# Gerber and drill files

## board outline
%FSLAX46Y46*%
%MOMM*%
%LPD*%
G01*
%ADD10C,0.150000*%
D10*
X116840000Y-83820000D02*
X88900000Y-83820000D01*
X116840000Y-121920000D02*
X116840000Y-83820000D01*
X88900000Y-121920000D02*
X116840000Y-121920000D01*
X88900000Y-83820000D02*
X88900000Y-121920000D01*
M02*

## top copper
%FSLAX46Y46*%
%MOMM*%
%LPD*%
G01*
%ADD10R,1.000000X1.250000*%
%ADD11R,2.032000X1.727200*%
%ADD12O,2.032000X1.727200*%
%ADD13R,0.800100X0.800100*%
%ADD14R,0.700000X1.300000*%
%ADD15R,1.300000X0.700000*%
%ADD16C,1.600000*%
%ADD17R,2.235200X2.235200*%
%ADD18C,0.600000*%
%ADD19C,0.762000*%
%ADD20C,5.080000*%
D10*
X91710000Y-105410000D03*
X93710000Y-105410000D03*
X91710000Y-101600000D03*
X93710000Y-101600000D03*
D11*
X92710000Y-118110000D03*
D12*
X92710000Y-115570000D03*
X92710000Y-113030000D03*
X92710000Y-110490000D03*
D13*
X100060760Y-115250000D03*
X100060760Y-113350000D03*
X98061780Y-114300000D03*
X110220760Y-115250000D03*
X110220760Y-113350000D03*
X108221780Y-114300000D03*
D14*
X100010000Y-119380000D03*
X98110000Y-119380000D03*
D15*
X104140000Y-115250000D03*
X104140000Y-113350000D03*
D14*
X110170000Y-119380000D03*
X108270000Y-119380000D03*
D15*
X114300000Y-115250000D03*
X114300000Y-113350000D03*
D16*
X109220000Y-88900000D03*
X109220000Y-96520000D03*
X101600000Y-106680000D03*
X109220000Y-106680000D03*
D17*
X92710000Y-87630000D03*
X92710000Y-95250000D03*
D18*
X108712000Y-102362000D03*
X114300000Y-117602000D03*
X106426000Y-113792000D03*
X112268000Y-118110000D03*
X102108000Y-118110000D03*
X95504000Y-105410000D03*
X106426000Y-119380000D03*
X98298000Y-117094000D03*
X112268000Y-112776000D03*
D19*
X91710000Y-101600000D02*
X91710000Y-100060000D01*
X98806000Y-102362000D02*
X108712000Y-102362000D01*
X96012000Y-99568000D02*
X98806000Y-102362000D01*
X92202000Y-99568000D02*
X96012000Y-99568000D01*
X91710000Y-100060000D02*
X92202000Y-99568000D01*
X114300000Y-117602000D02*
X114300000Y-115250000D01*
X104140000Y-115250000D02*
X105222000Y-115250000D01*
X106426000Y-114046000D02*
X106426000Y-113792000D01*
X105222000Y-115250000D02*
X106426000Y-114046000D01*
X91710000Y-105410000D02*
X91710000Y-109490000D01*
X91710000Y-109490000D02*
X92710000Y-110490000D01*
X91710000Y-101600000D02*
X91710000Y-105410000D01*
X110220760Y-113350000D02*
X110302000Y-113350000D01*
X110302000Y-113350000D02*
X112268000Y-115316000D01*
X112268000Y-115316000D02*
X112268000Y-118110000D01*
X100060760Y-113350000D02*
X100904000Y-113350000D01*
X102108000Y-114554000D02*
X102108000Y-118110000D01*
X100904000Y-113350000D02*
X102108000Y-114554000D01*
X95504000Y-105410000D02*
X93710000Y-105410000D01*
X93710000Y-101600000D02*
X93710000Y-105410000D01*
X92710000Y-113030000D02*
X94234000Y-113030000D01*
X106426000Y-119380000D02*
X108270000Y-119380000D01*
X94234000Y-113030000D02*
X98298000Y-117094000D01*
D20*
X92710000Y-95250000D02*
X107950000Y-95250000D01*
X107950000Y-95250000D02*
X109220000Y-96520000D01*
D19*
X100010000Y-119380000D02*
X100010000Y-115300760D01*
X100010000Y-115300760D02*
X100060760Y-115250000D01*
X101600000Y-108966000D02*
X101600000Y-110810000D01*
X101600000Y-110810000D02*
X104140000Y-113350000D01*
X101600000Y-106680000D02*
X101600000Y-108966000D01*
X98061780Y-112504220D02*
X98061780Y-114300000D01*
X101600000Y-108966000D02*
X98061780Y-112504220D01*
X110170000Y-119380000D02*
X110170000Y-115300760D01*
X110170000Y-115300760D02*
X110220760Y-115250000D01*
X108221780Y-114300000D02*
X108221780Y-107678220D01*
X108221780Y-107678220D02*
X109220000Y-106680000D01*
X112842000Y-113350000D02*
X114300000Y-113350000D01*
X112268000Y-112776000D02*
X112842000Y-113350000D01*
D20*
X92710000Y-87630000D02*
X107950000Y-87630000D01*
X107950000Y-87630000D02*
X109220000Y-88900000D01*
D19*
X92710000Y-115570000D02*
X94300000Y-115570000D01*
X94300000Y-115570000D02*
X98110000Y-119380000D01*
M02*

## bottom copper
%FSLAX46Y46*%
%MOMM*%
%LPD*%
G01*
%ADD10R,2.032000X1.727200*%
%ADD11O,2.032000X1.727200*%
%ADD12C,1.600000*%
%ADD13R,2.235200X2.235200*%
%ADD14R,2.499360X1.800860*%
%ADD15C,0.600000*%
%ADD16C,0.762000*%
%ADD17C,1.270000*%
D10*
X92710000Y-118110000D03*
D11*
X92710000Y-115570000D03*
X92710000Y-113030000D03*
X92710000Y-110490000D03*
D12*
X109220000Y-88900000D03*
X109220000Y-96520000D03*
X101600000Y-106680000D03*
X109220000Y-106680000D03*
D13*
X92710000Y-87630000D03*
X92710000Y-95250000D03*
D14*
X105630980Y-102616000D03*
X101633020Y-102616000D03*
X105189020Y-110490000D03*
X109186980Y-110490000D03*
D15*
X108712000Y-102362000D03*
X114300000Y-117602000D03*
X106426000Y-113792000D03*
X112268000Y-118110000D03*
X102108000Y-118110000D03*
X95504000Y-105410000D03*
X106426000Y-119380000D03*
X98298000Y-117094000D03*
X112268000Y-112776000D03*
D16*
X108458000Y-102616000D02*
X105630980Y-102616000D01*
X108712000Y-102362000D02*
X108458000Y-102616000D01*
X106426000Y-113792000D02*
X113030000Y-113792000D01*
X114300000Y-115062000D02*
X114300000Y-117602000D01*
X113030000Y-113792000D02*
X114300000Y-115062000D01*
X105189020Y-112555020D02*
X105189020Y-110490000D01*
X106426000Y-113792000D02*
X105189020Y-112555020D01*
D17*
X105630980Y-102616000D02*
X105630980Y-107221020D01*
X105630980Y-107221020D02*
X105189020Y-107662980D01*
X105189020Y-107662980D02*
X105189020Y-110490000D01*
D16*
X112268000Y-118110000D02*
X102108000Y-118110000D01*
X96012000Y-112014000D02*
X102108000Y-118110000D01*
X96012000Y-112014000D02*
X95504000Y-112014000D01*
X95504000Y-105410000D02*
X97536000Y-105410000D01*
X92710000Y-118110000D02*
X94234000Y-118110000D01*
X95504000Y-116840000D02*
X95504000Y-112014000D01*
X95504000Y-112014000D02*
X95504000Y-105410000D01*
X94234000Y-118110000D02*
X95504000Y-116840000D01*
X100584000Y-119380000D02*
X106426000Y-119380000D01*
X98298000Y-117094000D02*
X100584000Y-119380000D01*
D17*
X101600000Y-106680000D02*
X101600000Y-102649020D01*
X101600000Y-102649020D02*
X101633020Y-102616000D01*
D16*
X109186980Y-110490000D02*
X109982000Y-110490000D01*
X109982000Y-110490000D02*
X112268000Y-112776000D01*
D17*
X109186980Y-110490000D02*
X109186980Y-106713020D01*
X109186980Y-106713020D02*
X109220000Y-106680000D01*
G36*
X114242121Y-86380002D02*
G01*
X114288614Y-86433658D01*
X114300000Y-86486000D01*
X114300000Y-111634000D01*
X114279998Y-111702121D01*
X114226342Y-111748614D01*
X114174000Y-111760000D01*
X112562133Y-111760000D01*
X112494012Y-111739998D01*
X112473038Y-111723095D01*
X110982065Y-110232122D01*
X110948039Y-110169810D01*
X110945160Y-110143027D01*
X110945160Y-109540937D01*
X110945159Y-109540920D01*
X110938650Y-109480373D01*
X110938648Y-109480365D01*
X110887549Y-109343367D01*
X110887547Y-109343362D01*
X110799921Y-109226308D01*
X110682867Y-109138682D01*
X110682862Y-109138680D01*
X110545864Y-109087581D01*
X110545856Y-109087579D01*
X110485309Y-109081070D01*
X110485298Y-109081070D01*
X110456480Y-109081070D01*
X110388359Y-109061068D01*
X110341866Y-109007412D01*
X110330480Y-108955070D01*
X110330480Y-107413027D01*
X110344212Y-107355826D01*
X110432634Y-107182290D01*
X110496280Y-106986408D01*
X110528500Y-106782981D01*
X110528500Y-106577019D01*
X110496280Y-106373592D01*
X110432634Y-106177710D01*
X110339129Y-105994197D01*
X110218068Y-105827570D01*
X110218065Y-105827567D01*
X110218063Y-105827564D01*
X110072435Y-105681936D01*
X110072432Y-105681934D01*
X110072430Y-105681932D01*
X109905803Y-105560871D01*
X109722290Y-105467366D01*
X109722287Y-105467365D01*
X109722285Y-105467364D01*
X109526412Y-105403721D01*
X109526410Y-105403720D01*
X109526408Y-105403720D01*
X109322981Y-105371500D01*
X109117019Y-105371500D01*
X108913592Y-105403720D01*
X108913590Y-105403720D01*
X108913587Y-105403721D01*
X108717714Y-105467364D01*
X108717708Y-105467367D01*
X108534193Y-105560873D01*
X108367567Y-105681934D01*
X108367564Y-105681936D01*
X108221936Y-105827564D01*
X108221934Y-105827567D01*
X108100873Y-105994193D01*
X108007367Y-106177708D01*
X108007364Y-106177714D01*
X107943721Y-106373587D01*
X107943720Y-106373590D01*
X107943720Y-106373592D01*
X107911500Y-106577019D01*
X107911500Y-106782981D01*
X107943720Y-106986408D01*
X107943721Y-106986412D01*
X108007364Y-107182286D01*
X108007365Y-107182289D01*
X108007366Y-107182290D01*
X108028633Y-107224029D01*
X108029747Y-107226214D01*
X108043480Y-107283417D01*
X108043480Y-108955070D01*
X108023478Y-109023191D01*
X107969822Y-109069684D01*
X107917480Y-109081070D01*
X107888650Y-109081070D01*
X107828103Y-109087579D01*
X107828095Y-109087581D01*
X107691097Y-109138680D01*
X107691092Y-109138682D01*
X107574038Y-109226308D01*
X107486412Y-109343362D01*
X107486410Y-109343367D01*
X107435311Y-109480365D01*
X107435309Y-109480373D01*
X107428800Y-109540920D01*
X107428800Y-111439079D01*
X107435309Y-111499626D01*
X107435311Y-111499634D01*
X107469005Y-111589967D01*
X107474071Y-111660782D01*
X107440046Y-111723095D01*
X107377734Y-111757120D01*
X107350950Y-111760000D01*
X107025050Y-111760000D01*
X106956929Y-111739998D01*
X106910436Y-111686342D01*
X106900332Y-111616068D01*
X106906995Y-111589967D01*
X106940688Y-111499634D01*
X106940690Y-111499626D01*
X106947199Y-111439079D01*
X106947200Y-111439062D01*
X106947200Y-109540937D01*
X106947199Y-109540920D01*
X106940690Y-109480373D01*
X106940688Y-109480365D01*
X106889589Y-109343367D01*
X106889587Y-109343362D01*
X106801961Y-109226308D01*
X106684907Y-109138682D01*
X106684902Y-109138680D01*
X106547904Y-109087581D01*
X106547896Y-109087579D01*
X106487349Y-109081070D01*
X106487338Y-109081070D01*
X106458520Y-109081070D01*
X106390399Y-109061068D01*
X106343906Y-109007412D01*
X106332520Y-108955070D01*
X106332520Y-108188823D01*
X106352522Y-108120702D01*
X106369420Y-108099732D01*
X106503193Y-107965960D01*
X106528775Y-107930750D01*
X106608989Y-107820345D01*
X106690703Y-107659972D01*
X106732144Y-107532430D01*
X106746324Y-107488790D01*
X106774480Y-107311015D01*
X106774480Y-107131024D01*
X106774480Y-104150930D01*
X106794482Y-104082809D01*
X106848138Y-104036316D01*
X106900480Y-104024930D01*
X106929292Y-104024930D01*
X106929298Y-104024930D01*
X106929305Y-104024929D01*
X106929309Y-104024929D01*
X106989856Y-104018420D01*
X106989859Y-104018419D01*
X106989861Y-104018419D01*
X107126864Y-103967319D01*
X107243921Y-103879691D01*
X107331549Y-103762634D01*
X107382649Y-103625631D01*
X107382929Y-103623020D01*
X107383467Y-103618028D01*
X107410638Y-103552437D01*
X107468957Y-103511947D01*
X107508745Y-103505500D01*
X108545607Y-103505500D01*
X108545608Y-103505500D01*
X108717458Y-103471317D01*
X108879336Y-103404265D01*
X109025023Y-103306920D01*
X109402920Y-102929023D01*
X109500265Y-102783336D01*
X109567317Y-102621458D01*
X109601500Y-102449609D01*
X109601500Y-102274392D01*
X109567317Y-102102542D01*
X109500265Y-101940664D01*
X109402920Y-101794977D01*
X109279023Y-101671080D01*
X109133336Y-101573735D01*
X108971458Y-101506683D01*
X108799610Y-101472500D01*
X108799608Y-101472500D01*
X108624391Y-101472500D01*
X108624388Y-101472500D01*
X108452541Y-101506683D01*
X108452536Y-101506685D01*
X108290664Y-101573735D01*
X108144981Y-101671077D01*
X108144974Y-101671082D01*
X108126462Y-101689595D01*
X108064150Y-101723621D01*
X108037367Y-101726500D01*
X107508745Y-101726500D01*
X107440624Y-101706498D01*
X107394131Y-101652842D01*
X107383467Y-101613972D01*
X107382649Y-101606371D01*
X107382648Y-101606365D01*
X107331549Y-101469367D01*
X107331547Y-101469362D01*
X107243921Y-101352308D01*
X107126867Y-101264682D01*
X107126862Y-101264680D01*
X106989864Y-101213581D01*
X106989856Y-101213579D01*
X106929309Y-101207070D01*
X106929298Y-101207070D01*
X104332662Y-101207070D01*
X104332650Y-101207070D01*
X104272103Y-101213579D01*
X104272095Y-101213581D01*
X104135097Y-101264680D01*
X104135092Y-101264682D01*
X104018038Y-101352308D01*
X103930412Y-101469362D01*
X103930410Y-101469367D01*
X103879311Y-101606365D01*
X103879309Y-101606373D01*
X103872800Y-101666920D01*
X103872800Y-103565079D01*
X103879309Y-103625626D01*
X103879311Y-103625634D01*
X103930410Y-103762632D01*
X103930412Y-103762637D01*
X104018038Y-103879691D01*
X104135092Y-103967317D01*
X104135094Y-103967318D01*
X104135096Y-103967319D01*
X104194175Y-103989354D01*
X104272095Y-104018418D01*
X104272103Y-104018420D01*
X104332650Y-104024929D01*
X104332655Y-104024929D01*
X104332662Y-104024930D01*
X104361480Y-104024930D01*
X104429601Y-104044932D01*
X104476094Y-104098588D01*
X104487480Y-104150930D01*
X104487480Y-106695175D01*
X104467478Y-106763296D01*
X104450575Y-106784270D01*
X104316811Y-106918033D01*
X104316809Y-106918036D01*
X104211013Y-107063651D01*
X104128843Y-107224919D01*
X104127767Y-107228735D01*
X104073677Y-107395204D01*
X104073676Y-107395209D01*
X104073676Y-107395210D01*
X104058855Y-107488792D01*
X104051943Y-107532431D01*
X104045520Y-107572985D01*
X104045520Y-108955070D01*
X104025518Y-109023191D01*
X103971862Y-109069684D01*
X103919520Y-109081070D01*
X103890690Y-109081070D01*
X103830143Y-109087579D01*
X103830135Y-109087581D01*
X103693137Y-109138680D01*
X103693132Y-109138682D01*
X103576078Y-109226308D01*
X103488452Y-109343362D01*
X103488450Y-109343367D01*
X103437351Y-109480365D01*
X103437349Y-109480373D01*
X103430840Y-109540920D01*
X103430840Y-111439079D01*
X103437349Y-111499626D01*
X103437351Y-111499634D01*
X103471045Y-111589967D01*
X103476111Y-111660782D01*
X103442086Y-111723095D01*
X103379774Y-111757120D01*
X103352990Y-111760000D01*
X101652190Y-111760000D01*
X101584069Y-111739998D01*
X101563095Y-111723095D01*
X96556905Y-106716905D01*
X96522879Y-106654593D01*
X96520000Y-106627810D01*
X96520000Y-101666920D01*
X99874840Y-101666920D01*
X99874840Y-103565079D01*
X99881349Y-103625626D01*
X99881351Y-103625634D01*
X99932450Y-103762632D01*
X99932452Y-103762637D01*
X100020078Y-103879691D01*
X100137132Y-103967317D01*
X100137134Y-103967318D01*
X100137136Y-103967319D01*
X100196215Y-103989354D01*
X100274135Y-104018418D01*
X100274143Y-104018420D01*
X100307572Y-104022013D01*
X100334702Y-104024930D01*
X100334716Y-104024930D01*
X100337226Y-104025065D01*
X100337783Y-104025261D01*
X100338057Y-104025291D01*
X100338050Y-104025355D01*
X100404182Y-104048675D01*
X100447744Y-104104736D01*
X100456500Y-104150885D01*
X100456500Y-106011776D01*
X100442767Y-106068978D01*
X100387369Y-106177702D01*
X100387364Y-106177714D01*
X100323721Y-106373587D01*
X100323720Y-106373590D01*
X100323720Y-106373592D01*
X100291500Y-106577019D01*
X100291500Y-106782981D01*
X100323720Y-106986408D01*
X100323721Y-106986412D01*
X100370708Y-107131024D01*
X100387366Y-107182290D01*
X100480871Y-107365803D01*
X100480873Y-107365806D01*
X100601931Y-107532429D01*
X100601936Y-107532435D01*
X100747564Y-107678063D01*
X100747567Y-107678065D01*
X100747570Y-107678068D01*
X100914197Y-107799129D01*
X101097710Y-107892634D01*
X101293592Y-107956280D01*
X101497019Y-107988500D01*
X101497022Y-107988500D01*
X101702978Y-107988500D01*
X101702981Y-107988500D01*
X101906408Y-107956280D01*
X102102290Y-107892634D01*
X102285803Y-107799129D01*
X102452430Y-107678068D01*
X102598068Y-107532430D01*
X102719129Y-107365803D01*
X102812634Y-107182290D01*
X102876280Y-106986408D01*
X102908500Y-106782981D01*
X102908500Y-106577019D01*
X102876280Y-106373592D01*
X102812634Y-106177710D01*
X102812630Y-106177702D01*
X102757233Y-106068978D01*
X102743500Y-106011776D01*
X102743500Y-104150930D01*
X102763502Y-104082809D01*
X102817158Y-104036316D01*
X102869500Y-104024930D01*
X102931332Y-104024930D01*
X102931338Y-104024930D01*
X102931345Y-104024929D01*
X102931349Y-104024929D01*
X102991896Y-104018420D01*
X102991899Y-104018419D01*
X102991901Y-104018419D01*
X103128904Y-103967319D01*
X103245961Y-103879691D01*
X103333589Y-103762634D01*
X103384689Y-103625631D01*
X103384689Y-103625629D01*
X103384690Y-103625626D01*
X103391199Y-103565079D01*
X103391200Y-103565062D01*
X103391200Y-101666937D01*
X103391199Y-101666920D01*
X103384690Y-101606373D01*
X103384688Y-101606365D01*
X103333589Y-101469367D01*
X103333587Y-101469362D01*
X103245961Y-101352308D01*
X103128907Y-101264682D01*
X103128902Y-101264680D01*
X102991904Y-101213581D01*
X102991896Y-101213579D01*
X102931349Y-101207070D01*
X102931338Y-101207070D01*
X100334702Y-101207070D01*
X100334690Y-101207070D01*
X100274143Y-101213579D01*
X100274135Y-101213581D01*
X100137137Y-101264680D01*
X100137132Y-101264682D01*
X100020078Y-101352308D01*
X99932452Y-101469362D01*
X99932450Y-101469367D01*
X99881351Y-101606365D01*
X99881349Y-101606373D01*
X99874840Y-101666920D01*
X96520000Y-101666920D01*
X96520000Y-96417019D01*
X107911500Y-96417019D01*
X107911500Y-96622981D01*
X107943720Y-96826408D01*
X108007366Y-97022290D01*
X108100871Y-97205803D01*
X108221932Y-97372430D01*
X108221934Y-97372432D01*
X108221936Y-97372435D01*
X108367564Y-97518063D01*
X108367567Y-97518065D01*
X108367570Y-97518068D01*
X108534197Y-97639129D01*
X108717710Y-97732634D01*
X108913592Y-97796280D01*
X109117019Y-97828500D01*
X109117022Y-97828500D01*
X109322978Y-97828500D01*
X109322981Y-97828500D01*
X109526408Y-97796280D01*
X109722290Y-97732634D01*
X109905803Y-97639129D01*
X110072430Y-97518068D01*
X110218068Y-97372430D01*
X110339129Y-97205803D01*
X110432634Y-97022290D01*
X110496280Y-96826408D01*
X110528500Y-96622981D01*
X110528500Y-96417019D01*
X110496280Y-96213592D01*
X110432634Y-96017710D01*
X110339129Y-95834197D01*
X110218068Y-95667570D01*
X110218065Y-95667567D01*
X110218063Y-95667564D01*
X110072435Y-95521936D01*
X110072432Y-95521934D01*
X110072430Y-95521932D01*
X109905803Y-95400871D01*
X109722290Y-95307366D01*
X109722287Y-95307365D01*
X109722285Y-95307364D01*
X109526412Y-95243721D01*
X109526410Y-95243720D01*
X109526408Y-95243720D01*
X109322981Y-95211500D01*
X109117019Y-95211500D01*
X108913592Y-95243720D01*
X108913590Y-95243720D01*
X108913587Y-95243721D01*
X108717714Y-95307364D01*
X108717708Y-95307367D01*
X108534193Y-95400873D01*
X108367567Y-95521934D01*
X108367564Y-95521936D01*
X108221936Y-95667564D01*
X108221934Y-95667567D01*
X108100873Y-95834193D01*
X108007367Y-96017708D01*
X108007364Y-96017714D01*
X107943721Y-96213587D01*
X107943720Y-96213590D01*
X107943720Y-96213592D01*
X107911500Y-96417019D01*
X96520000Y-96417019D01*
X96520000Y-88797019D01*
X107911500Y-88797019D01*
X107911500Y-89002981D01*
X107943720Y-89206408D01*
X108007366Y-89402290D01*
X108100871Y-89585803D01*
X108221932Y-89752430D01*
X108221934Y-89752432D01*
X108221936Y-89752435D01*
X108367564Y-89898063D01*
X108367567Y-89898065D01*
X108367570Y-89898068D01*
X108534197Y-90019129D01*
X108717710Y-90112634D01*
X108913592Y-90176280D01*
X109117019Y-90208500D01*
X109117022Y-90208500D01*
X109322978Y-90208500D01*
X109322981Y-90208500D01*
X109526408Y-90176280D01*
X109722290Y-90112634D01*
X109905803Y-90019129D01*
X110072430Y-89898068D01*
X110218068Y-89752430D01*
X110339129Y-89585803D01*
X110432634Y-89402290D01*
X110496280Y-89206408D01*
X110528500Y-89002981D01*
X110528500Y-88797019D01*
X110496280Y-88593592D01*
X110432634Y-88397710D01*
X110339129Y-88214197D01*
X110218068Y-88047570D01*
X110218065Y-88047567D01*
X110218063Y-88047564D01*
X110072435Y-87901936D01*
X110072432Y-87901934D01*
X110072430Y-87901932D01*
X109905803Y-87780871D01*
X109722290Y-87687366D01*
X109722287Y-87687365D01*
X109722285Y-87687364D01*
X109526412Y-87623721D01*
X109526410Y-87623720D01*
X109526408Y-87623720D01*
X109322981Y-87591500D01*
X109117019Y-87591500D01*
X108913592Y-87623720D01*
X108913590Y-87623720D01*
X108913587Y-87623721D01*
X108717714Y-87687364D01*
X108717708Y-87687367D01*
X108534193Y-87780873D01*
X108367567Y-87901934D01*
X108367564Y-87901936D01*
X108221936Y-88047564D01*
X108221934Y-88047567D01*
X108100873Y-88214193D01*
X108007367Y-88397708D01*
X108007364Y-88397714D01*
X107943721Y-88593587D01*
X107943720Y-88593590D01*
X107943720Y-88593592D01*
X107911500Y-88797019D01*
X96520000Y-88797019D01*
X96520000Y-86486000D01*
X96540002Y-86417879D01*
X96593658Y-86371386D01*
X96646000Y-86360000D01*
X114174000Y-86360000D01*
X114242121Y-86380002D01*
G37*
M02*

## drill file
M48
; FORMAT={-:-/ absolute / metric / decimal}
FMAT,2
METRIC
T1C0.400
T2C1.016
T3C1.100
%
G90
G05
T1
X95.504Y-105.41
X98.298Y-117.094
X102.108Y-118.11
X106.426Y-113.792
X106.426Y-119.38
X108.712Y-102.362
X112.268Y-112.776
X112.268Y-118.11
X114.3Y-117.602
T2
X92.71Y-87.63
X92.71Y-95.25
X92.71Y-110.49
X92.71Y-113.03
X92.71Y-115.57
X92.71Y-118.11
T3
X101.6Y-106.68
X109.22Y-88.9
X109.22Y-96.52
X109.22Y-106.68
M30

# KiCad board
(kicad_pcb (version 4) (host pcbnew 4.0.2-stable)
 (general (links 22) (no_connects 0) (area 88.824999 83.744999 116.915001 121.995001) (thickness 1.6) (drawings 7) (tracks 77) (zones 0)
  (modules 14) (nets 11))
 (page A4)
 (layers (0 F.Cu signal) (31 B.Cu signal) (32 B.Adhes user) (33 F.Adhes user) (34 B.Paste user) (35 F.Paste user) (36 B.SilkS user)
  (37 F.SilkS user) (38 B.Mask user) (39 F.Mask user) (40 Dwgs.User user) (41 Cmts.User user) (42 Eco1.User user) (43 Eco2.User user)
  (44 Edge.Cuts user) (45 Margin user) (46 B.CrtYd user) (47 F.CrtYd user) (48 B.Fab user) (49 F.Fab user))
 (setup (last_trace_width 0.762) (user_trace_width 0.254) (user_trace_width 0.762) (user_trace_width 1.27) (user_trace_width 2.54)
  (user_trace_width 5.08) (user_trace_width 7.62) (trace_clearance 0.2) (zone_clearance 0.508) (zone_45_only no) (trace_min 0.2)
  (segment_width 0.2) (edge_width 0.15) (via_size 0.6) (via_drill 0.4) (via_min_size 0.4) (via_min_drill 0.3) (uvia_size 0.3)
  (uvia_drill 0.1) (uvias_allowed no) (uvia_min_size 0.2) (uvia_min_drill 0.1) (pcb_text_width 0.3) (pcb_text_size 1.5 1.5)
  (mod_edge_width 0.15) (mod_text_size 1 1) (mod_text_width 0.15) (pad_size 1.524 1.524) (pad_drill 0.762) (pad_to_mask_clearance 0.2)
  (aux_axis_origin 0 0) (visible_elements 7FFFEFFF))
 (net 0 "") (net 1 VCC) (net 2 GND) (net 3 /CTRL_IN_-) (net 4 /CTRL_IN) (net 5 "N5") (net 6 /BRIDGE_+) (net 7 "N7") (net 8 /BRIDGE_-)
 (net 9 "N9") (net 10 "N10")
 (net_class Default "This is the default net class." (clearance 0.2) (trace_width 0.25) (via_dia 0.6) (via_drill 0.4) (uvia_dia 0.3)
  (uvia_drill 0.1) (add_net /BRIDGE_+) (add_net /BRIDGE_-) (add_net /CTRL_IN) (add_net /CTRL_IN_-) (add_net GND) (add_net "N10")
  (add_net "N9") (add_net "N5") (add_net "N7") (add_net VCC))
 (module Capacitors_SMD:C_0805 (layer F.Cu) (at 92.71 105.41)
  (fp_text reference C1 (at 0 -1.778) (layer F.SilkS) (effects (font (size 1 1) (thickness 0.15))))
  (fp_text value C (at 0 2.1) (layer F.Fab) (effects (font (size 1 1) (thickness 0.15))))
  (pad 1 smd rect (at -1 0) (size 1 1.25) (layers F.Cu F.Paste F.Mask) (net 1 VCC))
  (pad 2 smd rect (at 1 0) (size 1 1.25) (layers F.Cu F.Paste F.Mask) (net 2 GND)))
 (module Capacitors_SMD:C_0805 (layer F.Cu) (at 92.71 101.6)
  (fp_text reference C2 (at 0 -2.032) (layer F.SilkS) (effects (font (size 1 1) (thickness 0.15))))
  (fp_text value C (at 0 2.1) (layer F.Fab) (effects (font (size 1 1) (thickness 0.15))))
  (pad 1 smd rect (at -1 0) (size 1 1.25) (layers F.Cu F.Paste F.Mask) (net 1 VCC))
  (pad 2 smd rect (at 1 0) (size 1 1.25) (layers F.Cu F.Paste F.Mask) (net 2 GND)))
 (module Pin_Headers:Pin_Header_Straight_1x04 (layer F.Cu) (at 92.71 118.11 180)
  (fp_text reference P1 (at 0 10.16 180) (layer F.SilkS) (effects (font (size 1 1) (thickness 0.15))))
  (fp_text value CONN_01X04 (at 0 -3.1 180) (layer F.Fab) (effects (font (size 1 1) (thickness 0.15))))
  (pad 1 thru_hole rect (at 0 0 180) (size 2.032 1.7272) (drill 1.016) (layers *.Cu *.Mask F.SilkS) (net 2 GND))
  (pad 2 thru_hole oval (at 0 2.54 180) (size 2.032 1.7272) (drill 1.016) (layers *.Cu *.Mask F.SilkS) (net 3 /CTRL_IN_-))
  (pad 3 thru_hole oval (at 0 5.08 180) (size 2.032 1.7272) (drill 1.016) (layers *.Cu *.Mask F.SilkS) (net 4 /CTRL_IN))
  (pad 4 thru_hole oval (at 0 7.62 180) (size 2.032 1.7272) (drill 1.016) (layers *.Cu *.Mask F.SilkS) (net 1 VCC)))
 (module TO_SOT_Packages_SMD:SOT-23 (layer F.Cu) (at 99.06 114.3 90)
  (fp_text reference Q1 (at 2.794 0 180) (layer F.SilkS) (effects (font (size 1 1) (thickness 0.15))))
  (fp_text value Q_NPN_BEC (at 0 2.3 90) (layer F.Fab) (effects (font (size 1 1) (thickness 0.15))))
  (pad 1 smd rect (at -0.95 1.00076 90) (size 0.8001 0.8001) (layers F.Cu F.Paste F.Mask) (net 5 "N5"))
  (pad 2 smd rect (at 0.95 1.00076 90) (size 0.8001 0.8001) (layers F.Cu F.Paste F.Mask) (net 2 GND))
  (pad 3 smd rect (at 0 -0.99822 90) (size 0.8001 0.8001) (layers F.Cu F.Paste F.Mask) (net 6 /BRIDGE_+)))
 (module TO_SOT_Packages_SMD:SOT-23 (layer F.Cu) (at 109.22 114.3 90)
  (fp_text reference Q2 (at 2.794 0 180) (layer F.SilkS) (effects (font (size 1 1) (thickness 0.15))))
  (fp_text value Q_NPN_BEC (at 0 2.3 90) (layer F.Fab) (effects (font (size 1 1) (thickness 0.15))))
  (pad 1 smd rect (at -0.95 1.00076 90) (size 0.8001 0.8001) (layers F.Cu F.Paste F.Mask) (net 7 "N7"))
  (pad 2 smd rect (at 0.95 1.00076 90) (size 0.8001 0.8001) (layers F.Cu F.Paste F.Mask) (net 2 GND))
  (pad 3 smd rect (at 0 -0.99822 90) (size 0.8001 0.8001) (layers F.Cu F.Paste F.Mask) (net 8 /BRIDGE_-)))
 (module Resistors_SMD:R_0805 (layer F.Cu) (at 99.06 119.38 180)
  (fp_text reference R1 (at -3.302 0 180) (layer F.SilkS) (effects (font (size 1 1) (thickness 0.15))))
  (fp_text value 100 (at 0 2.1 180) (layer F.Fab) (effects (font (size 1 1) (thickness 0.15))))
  (pad 1 smd rect (at -0.95 0 180) (size 0.7 1.3) (layers F.Cu F.Paste F.Mask) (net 5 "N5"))
  (pad 2 smd rect (at 0.95 0 180) (size 0.7 1.3) (layers F.Cu F.Paste F.Mask) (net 3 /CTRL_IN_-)))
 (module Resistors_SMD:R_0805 (layer F.Cu) (at 104.14 114.3 90)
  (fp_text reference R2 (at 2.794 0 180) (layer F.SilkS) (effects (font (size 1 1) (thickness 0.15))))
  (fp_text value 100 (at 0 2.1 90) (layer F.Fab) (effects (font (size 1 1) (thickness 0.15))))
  (pad 1 smd rect (at -0.95 0 90) (size 0.7 1.3) (layers F.Cu F.Paste F.Mask) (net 1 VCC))
  (pad 2 smd rect (at 0.95 0 90) (size 0.7 1.3) (layers F.Cu F.Paste F.Mask) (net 6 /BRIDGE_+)))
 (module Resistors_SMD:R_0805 (layer F.Cu) (at 109.22 119.38 180)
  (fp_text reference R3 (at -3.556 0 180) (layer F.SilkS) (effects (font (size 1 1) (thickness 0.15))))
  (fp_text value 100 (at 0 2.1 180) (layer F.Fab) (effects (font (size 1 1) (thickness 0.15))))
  (pad 1 smd rect (at -0.95 0 180) (size 0.7 1.3) (layers F.Cu F.Paste F.Mask) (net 7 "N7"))
  (pad 2 smd rect (at 0.95 0 180) (size 0.7 1.3) (layers F.Cu F.Paste F.Mask) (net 4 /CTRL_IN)))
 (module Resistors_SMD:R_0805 (layer F.Cu) (at 114.3 114.3 90)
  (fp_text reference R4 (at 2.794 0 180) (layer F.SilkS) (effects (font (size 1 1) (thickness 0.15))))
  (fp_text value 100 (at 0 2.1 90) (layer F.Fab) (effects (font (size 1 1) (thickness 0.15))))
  (pad 1 smd rect (at -0.95 0 90) (size 0.7 1.3) (layers F.Cu F.Paste F.Mask) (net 1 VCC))
  (pad 2 smd rect (at 0.95 0 90) (size 0.7 1.3) (layers F.Cu F.Paste F.Mask) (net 8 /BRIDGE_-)))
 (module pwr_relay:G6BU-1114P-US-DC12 (layer F.Cu) (at 109.22 106.68 90)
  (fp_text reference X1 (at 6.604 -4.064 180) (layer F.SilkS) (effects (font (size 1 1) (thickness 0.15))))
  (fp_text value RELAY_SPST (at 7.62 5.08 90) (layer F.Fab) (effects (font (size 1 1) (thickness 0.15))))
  (pad 4 thru_hole circle (at 17.78 0 90) (size 1.6 1.6) (drill 1.1) (layers *.Cu *.Mask F.SilkS) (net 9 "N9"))
  (pad 3 thru_hole circle (at 10.16 0 90) (size 1.6 1.6) (drill 1.1) (layers *.Cu *.Mask F.SilkS) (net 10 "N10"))
  (pad 6 thru_hole circle (at 0 -7.62 90) (size 1.6 1.6) (drill 1.1) (layers *.Cu *.Mask F.SilkS) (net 6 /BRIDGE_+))
  (pad 1 thru_hole circle (at 0 0 90) (size 1.6 1.6) (drill 1.1) (layers *.Cu *.Mask F.SilkS) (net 8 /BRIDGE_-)))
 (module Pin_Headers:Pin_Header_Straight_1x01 (layer F.Cu) (at 92.71 87.63)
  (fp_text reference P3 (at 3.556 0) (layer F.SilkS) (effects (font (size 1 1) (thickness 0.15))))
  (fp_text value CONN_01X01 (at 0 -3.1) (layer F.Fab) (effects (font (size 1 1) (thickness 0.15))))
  (pad 1 thru_hole rect (at 0 0) (size 2.2352 2.2352) (drill 1.016) (layers *.Cu *.Mask F.SilkS) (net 9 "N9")))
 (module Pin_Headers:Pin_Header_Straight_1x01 (layer F.Cu) (at 92.71 95.25)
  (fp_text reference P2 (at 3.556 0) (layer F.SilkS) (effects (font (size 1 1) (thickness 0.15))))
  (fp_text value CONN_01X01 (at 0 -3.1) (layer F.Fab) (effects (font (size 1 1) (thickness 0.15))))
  (pad 1 thru_hole rect (at 0 0) (size 2.2352 2.2352) (drill 1.016) (layers *.Cu *.Mask F.SilkS) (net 10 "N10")))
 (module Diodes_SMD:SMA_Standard (layer B.Cu) (at 103.632 102.616 180)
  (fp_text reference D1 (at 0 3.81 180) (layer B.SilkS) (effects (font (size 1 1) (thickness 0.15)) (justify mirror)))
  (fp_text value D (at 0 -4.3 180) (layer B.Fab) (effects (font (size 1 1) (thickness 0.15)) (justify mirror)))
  (pad 1 smd rect (at -1.99898 0 180) (size 2.49936 1.80086) (layers B.Cu B.Paste B.Mask) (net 1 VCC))
  (pad 2 smd rect (at 1.99898 0 180) (size 2.49936 1.80086) (layers B.Cu B.Paste B.Mask) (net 6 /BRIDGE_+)))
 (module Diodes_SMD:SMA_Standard (layer B.Cu) (at 107.188 110.49)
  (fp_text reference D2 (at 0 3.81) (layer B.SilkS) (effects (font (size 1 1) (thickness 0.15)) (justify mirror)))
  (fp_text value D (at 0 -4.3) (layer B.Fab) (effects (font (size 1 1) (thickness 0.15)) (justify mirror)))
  (pad 1 smd rect (at -1.99898 0) (size 2.49936 1.80086) (layers B.Cu B.Paste B.Mask) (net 1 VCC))
  (pad 2 smd rect (at 1.99898 0) (size 2.49936 1.80086) (layers B.Cu B.Paste B.Mask) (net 8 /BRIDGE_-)))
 (gr_line (start 116.84 83.82) (end 88.9 83.82) (angle 90) (layer Edge.Cuts) (width 0.15))
 (gr_line (start 116.84 121.92) (end 116.84 83.82) (angle 90) (layer Edge.Cuts) (width 0.15))
 (gr_line (start 88.9 121.92) (end 116.84 121.92) (angle 90) (layer Edge.Cuts) (width 0.15))
 (gr_line (start 88.9 83.82) (end 88.9 121.92) (angle 90) (layer Edge.Cuts) (width 0.15))
 (segment (start 91.71 101.6) (end 91.71 100.06) (width 0.762) (layer F.Cu) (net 1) (status 400000))
 (segment (start 108.458 102.616) (end 105.63098 102.616) (width 0.762) (layer B.Cu) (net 1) (status 800000))
 (segment (start 108.712 102.362) (end 108.458 102.616) (width 0.762) (layer B.Cu) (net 1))
 (via (at 108.712 102.362) (size 0.6) (drill 0.4) (layers F.Cu B.Cu) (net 1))
 (segment (start 98.806 102.362) (end 108.712 102.362) (width 0.762) (layer F.Cu) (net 1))
 (segment (start 96.012 99.568) (end 98.806 102.362) (width 0.762) (layer F.Cu) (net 1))
 (segment (start 92.202 99.568) (end 96.012 99.568) (width 0.762) (layer F.Cu) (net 1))
 (segment (start 91.71 100.06) (end 92.202 99.568) (width 0.762) (layer F.Cu) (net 1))
 (segment (start 106.426 113.792) (end 113.03 113.792) (width 0.762) (layer B.Cu) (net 1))
 (segment (start 114.3 117.602) (end 114.3 115.25) (width 0.762) (layer F.Cu) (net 1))
 (via (at 114.3 117.602) (size 0.6) (drill 0.4) (layers F.Cu B.Cu) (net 1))
 (segment (start 114.3 115.062) (end 114.3 117.602) (width 0.762) (layer B.Cu) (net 1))
 (segment (start 113.03 113.792) (end 114.3 115.062) (width 0.762) (layer B.Cu) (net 1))
 (segment (start 104.14 115.25) (end 105.222 115.25) (width 0.762) (layer F.Cu) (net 1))
 (segment (start 105.18902 112.55502) (end 105.18902 110.49) (width 0.762) (layer B.Cu) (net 1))
 (segment (start 106.426 113.792) (end 105.18902 112.55502) (width 0.762) (layer B.Cu) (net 1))
 (via (at 106.426 113.792) (size 0.6) (drill 0.4) (layers F.Cu B.Cu) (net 1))
 (segment (start 106.426 114.046) (end 106.426 113.792) (width 0.762) (layer F.Cu) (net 1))
 (segment (start 105.222 115.25) (end 106.426 114.046) (width 0.762) (layer F.Cu) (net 1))
 (segment (start 105.63098 102.616) (end 105.63098 107.22102) (width 1.27) (layer B.Cu) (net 1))
 (segment (start 105.63098 107.22102) (end 105.18902 107.66298) (width 1.27) (layer B.Cu) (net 1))
 (segment (start 105.18902 107.66298) (end 105.18902 110.49) (width 1.27) (layer B.Cu) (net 1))
 (segment (start 91.71 105.41) (end 91.71 109.49) (width 0.762) (layer F.Cu) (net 1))
 (segment (start 91.71 109.49) (end 92.71 110.49) (width 0.762) (layer F.Cu) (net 1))
 (segment (start 91.71 101.6) (end 91.71 105.41) (width 0.762) (layer F.Cu) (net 1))
 (segment (start 110.22076 113.35) (end 110.302 113.35) (width 0.762) (layer F.Cu) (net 2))
 (segment (start 110.302 113.35) (end 112.268 115.316) (width 0.762) (layer F.Cu) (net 2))
 (segment (start 112.268 115.316) (end 112.268 118.11) (width 0.762) (layer F.Cu) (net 2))
 (via (at 112.268 118.11) (size 0.6) (drill 0.4) (layers F.Cu B.Cu) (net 2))
 (segment (start 112.268 118.11) (end 102.108 118.11) (width 0.762) (layer B.Cu) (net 2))
 (segment (start 100.06076 113.35) (end 100.904 113.35) (width 0.762) (layer F.Cu) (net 2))
 (segment (start 96.012 112.014) (end 102.108 118.11) (width 0.762) (layer B.Cu) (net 2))
 (via (at 102.108 118.11) (size 0.6) (drill 0.4) (layers F.Cu B.Cu) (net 2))
 (segment (start 96.012 112.014) (end 95.504 112.014) (width 0.762) (layer B.Cu) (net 2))
 (segment (start 102.108 114.554) (end 102.108 118.11) (width 0.762) (layer F.Cu) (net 2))
 (segment (start 100.904 113.35) (end 102.108 114.554) (width 0.762) (layer F.Cu) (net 2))
 (segment (start 95.504 105.41) (end 97.536 105.41) (width 0.762) (layer B.Cu) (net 2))
 (segment (start 92.71 118.11) (end 94.234 118.11) (width 0.762) (layer B.Cu) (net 2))
 (segment (start 95.504 105.41) (end 93.71 105.41) (width 0.762) (layer F.Cu) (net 2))
 (via (at 95.504 105.41) (size 0.6) (drill 0.4) (layers F.Cu B.Cu) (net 2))
 (segment (start 95.504 116.84) (end 95.504 112.014) (width 0.762) (layer B.Cu) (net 2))
 (segment (start 95.504 112.014) (end 95.504 105.41) (width 0.762) (layer B.Cu) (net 2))
 (segment (start 94.234 118.11) (end 95.504 116.84) (width 0.762) (layer B.Cu) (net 2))
 (segment (start 93.71 101.6) (end 93.71 105.41) (width 0.762) (layer F.Cu) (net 2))
 (segment (start 92.71 113.03) (end 94.234 113.03) (width 0.762) (layer F.Cu) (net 4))
 (segment (start 106.426 119.38) (end 108.27 119.38) (width 0.762) (layer F.Cu) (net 4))
 (via (at 106.426 119.38) (size 0.6) (drill 0.4) (layers F.Cu B.Cu) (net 4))
 (segment (start 100.584 119.38) (end 106.426 119.38) (width 0.762) (layer B.Cu) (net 4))
 (segment (start 98.298 117.094) (end 100.584 119.38) (width 0.762) (layer B.Cu) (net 4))
 (via (at 98.298 117.094) (size 0.6) (drill 0.4) (layers F.Cu B.Cu) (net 4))
 (segment (start 94.234 113.03) (end 98.298 117.094) (width 0.762) (layer F.Cu) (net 4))
 (segment (start 92.71 95.25) (end 107.95 95.25) (width 5.08) (layer F.Cu) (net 10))
 (segment (start 107.95 95.25) (end 109.22 96.52) (width 5.08) (layer F.Cu) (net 10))
 (segment (start 100.01 119.38) (end 100.01 115.30076) (width 0.762) (layer F.Cu) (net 5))
 (segment (start 100.01 115.30076) (end 100.06076 115.25) (width 0.762) (layer F.Cu) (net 5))
 (segment (start 101.6 108.966) (end 101.6 110.81) (width 0.762) (layer F.Cu) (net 6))
 (segment (start 101.6 110.81) (end 104.14 113.35) (width 0.762) (layer F.Cu) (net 6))
 (segment (start 101.6 106.68) (end 101.6 108.966) (width 0.762) (layer F.Cu) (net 6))
 (segment (start 98.06178 112.50422) (end 98.06178 114.3) (width 0.762) (layer F.Cu) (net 6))
 (segment (start 101.6 108.966) (end 98.06178 112.50422) (width 0.762) (layer F.Cu) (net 6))
 (segment (start 101.6 106.68) (end 101.6 102.64902) (width 1.27) (layer B.Cu) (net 6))
 (segment (start 101.6 102.64902) (end 101.63302 102.616) (width 1.27) (layer B.Cu) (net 6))
 (segment (start 110.17 119.38) (end 110.17 115.30076) (width 0.762) (layer F.Cu) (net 7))
 (segment (start 110.17 115.30076) (end 110.22076 115.25) (width 0.762) (layer F.Cu) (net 7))
 (segment (start 108.22178 114.3) (end 108.22178 107.67822) (width 0.762) (layer F.Cu) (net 8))
 (segment (start 108.22178 107.67822) (end 109.22 106.68) (width 0.762) (layer F.Cu) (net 8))
 (segment (start 109.18698 110.49) (end 109.982 110.49) (width 0.762) (layer B.Cu) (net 8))
 (segment (start 109.982 110.49) (end 112.268 112.776) (width 0.762) (layer B.Cu) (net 8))
 (segment (start 112.842 113.35) (end 114.3 113.35) (width 0.762) (layer F.Cu) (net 8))
 (segment (start 112.268 112.776) (end 112.842 113.35) (width 0.762) (layer F.Cu) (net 8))
 (via (at 112.268 112.776) (size 0.6) (drill 0.4) (layers F.Cu B.Cu) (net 8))
 (segment (start 109.18698 110.49) (end 109.18698 106.71302) (width 1.27) (layer B.Cu) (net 8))
 (segment (start 109.18698 106.71302) (end 109.22 106.68) (width 1.27) (layer B.Cu) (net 8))
 (segment (start 92.71 87.63) (end 107.95 87.63) (width 5.08) (layer F.Cu) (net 9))
 (segment (start 107.95 87.63) (end 109.22 88.9) (width 5.08) (layer F.Cu) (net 9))
 (segment (start 92.71 115.57) (end 94.3 115.57) (width 0.762) (layer F.Cu) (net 3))
 (segment (start 94.3 115.57) (end 98.11 119.38) (width 0.762) (layer F.Cu) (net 3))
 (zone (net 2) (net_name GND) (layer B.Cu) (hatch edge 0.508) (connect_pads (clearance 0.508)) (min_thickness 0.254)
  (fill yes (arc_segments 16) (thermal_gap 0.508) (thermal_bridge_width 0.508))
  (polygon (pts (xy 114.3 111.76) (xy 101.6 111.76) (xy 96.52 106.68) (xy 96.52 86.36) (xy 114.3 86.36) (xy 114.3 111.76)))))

